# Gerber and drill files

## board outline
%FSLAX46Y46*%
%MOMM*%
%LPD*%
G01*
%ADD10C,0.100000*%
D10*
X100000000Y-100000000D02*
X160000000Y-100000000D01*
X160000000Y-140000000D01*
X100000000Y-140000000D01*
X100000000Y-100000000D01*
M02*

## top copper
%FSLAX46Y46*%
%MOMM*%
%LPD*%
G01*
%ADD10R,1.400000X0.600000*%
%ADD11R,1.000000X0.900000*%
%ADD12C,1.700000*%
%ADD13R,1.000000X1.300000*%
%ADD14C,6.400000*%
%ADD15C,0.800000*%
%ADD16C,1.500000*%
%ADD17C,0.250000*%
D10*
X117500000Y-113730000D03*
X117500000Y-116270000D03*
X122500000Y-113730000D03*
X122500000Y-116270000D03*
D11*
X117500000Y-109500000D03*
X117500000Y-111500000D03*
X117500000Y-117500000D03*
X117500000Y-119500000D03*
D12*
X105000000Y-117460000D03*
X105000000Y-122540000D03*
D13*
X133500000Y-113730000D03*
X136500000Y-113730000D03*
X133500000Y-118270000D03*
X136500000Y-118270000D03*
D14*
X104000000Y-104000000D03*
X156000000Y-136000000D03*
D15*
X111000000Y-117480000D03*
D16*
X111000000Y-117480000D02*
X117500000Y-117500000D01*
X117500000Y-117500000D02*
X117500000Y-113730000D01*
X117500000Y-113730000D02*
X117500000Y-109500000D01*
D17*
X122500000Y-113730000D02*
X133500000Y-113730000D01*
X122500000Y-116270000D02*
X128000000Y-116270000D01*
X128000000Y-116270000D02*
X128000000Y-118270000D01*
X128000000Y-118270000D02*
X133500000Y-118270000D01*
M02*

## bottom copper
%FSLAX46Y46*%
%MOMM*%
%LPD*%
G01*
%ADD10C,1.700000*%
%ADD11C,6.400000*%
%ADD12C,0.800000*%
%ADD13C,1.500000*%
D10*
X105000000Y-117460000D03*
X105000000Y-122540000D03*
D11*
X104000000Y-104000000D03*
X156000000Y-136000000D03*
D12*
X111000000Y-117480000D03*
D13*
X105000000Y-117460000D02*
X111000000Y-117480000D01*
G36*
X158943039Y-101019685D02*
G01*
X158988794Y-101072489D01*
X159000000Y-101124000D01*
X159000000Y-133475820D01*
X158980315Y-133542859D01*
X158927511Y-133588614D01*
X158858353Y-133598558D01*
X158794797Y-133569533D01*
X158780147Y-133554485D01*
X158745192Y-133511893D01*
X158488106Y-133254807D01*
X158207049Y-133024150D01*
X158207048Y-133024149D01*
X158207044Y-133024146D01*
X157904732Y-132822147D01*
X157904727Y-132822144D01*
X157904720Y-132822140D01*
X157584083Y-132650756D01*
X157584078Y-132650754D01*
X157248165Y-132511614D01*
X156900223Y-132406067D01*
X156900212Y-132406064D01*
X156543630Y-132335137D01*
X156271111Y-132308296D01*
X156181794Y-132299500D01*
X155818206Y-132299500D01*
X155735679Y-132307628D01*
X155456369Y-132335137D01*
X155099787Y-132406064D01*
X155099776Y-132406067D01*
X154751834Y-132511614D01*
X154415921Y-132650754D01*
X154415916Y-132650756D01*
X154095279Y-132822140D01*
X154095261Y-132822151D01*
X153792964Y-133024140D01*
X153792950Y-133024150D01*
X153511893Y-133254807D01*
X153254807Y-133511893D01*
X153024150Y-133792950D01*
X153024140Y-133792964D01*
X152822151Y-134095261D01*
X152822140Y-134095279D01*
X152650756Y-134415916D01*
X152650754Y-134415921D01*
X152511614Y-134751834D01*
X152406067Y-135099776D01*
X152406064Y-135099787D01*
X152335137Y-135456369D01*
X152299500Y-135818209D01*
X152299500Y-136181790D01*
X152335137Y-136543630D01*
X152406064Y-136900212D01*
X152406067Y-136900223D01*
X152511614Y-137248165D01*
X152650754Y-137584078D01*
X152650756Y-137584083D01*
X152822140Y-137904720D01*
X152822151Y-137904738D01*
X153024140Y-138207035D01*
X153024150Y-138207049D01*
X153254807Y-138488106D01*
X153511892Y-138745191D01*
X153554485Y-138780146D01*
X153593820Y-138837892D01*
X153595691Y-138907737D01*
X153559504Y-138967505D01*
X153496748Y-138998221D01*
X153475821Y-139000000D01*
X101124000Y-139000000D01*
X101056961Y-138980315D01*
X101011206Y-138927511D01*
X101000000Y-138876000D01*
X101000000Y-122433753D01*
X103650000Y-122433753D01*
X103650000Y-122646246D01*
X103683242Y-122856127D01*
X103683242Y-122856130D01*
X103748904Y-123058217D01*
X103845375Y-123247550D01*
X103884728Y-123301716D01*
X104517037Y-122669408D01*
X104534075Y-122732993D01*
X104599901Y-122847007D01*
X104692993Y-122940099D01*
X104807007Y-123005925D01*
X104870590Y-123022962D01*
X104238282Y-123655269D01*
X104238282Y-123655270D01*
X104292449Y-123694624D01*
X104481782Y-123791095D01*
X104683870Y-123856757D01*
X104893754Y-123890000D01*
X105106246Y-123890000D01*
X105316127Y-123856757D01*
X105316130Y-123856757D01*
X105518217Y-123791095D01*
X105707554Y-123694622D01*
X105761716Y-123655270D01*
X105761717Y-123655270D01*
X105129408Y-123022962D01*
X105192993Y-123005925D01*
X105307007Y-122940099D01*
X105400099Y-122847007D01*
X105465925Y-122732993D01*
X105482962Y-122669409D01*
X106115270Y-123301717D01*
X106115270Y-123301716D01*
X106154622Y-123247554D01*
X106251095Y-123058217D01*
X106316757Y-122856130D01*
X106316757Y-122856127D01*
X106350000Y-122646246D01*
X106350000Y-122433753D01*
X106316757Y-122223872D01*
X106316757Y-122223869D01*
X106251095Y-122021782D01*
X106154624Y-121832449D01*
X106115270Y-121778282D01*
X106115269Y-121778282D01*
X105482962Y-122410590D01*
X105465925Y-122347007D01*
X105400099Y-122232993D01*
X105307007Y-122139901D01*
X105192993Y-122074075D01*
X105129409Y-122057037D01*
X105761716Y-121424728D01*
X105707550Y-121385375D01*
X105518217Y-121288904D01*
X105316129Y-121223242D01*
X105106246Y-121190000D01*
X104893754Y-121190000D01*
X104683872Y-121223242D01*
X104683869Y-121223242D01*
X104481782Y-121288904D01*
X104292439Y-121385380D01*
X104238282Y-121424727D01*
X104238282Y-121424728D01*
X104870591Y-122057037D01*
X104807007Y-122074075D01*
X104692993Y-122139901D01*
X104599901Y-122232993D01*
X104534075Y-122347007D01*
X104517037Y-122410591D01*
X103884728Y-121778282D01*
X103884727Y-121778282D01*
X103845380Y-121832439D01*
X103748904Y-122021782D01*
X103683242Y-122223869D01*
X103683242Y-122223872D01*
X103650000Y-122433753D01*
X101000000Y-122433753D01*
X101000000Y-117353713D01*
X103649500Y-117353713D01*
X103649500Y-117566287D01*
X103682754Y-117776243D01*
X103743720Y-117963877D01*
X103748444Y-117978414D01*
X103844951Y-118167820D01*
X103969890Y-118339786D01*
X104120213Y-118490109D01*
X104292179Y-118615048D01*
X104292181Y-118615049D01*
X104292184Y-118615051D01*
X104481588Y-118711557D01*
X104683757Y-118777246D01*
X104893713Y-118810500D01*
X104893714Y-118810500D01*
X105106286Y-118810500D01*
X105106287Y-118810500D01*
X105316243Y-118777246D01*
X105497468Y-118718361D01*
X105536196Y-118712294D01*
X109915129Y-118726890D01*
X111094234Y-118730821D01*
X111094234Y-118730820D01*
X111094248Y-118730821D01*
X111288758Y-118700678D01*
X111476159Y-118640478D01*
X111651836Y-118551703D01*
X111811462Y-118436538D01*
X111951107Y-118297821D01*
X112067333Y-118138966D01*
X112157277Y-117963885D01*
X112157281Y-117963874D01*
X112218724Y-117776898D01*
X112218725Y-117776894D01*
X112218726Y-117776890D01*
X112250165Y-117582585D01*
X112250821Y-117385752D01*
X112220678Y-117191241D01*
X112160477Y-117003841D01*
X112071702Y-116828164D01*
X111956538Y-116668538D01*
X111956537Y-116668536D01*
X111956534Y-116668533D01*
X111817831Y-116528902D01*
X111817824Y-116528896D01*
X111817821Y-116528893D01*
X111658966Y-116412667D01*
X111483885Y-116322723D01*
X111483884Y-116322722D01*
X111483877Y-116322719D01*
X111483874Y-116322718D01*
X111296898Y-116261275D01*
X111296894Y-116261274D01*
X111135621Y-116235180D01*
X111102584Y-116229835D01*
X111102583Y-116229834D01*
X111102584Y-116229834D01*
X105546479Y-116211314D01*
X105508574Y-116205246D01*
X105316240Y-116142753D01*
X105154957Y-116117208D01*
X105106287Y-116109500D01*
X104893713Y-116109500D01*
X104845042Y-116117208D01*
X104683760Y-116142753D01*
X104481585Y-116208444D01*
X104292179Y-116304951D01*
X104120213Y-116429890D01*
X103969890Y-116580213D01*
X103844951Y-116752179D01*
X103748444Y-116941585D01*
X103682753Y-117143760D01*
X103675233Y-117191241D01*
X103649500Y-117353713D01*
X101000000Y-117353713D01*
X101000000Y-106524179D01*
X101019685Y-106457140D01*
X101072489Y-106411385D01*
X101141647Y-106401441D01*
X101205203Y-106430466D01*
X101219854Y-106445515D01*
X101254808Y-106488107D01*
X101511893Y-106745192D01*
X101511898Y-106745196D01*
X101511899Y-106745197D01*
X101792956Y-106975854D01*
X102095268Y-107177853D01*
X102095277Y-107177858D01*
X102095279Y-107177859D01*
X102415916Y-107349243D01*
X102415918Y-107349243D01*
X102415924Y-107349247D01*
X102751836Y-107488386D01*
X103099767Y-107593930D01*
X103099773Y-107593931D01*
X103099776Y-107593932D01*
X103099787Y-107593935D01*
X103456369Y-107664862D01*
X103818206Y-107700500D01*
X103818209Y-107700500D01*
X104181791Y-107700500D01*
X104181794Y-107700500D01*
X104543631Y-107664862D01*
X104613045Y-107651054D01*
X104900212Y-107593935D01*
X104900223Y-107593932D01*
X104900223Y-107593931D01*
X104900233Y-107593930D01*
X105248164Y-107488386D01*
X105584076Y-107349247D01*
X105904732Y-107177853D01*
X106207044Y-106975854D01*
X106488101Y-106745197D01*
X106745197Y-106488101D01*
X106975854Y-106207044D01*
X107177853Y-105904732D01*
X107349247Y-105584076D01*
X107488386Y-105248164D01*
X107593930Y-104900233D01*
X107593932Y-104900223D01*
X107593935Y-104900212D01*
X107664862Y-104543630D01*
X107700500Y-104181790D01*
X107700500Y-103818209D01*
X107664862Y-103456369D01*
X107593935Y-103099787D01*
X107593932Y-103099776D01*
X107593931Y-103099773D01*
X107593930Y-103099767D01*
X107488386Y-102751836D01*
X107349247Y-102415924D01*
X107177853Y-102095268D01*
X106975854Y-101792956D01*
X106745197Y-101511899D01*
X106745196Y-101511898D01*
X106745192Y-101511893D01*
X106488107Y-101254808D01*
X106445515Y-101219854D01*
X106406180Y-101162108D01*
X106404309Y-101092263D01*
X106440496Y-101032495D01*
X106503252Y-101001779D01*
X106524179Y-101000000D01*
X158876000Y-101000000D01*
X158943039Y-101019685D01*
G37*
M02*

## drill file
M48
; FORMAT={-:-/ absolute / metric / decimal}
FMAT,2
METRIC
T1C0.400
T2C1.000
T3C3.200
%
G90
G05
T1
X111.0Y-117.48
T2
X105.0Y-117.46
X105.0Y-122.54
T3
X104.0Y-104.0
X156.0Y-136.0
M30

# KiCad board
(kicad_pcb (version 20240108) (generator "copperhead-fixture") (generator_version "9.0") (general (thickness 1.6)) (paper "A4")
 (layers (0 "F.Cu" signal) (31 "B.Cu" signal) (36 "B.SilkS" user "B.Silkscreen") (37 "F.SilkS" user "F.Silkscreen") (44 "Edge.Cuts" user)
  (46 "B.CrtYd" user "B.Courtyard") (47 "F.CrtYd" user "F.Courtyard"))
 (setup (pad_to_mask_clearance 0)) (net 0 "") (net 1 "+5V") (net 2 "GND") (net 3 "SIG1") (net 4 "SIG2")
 (gr_rect (start 100 100) (end 160 140) (stroke (width 0.1) (type default)) (layer "Edge.Cuts"))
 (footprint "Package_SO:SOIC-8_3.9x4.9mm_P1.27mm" (layer "F.Cu") (at 120 115)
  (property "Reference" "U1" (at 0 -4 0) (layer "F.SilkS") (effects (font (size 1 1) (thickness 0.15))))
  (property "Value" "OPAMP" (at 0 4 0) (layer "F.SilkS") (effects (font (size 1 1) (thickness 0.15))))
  (pad "1" smd rect (at -2.5 -1.27) (size 1.4 0.6) (layers "F.Cu" "F.Mask" "F.Paste") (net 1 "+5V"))
  (pad "2" smd rect (at -2.5 1.27) (size 1.4 0.6) (layers "F.Cu" "F.Mask" "F.Paste") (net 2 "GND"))
  (pad "3" smd rect (at 2.5 -1.27) (size 1.4 0.6) (layers "F.Cu" "F.Mask" "F.Paste") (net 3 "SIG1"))
  (pad "4" smd rect (at 2.5 1.27) (size 1.4 0.6) (layers "F.Cu" "F.Mask" "F.Paste") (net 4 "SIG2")))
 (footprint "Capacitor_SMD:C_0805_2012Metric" (layer "F.Cu") (at 117.5 110.5)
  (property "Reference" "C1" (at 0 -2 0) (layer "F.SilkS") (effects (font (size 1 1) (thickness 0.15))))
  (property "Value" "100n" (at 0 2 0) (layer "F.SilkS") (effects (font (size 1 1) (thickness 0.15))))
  (pad "1" smd rect (at 0 -1) (size 1 0.9) (layers "F.Cu" "F.Mask" "F.Paste") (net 1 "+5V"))
  (pad "2" smd rect (at 0 1) (size 1 0.9) (layers "F.Cu" "F.Mask" "F.Paste") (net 2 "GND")))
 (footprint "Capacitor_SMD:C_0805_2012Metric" (layer "F.Cu") (at 117.5 118.5)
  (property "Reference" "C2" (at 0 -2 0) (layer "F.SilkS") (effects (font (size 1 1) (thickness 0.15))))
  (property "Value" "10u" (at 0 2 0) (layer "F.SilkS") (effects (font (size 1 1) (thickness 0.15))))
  (pad "1" smd rect (at 0 -1) (size 1 0.9) (layers "F.Cu" "F.Mask" "F.Paste") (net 1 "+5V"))
  (pad "2" smd rect (at 0 1) (size 1 0.9) (layers "F.Cu" "F.Mask" "F.Paste") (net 2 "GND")))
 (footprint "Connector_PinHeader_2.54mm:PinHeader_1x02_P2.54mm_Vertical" (layer "F.Cu") (at 105 120)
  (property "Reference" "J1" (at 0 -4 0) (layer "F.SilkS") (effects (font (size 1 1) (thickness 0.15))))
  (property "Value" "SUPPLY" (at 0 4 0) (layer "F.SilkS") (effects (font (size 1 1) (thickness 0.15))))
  (pad "1" thru_hole circle (at 0 -2.54) (size 1.7 1.7) (drill 1) (layers "*.Cu" "*.Mask") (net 1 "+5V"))
  (pad "2" thru_hole circle (at 0 2.54) (size 1.7 1.7) (drill 1) (layers "*.Cu" "*.Mask") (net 2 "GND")))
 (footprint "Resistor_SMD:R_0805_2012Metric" (layer "F.Cu") (at 135 113.73)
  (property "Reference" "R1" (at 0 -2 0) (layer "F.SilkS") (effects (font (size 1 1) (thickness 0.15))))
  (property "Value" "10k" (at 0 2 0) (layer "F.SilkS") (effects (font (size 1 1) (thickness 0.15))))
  (pad "1" smd rect (at -1.5 0) (size 1 1.3) (layers "F.Cu" "F.Mask" "F.Paste") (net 3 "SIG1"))
  (pad "2" smd rect (at 1.5 0) (size 1 1.3) (layers "F.Cu" "F.Mask" "F.Paste") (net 2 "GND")))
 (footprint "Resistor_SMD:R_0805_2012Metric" (layer "F.Cu") (at 135 118.27)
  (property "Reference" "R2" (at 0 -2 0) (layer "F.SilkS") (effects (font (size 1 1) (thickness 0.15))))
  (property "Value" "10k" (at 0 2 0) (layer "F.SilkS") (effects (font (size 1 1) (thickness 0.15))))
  (pad "1" smd rect (at -1.5 0) (size 1 1.3) (layers "F.Cu" "F.Mask" "F.Paste") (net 4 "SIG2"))
  (pad "2" smd rect (at 1.5 0) (size 1 1.3) (layers "F.Cu" "F.Mask" "F.Paste") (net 2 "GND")))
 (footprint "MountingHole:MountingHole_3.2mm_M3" (layer "F.Cu") (at 104 104)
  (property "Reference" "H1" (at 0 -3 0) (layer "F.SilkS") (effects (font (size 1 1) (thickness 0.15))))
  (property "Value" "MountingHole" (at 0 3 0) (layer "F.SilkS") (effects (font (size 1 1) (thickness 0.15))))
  (pad "1" thru_hole circle (at 0 0) (size 6.4 6.4) (drill 3.2) (layers "*.Cu" "*.Mask")))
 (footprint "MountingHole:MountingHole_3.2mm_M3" (layer "F.Cu") (at 156 136)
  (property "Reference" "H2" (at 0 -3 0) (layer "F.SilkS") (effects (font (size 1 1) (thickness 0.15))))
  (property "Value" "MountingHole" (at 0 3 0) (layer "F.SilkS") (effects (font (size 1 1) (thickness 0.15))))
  (pad "1" thru_hole circle (at 0 0) (size 6.4 6.4) (drill 3.2) (layers "*.Cu" "*.Mask")))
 (segment (start 105 117.46) (end 111 117.48) (width 1.5) (layer "B.Cu") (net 1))
 (segment (start 111 117.48) (end 117.5 117.5) (width 1.5) (layer "F.Cu") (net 1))
 (segment (start 117.5 117.5) (end 117.5 113.73) (width 1.5) (layer "F.Cu") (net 1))
 (segment (start 117.5 113.73) (end 117.5 109.5) (width 1.5) (layer "F.Cu") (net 1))
 (segment (start 122.5 113.73) (end 133.5 113.73) (width 0.25) (layer "F.Cu") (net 3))
 (segment (start 122.5 116.27) (end 128 116.27) (width 0.25) (layer "F.Cu") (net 4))
 (segment (start 128 116.27) (end 128 118.27) (width 0.25) (layer "F.Cu") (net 4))
 (segment (start 128 118.27) (end 133.5 118.27) (width 0.25) (layer "F.Cu") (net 4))
 (via (at 111 117.48) (size 0.8) (drill 0.4) (layers "F.Cu" "B.Cu") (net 1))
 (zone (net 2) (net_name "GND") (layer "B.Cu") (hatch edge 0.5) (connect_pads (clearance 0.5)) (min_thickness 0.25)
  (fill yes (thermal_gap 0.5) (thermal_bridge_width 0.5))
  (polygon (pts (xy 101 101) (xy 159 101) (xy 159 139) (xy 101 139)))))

